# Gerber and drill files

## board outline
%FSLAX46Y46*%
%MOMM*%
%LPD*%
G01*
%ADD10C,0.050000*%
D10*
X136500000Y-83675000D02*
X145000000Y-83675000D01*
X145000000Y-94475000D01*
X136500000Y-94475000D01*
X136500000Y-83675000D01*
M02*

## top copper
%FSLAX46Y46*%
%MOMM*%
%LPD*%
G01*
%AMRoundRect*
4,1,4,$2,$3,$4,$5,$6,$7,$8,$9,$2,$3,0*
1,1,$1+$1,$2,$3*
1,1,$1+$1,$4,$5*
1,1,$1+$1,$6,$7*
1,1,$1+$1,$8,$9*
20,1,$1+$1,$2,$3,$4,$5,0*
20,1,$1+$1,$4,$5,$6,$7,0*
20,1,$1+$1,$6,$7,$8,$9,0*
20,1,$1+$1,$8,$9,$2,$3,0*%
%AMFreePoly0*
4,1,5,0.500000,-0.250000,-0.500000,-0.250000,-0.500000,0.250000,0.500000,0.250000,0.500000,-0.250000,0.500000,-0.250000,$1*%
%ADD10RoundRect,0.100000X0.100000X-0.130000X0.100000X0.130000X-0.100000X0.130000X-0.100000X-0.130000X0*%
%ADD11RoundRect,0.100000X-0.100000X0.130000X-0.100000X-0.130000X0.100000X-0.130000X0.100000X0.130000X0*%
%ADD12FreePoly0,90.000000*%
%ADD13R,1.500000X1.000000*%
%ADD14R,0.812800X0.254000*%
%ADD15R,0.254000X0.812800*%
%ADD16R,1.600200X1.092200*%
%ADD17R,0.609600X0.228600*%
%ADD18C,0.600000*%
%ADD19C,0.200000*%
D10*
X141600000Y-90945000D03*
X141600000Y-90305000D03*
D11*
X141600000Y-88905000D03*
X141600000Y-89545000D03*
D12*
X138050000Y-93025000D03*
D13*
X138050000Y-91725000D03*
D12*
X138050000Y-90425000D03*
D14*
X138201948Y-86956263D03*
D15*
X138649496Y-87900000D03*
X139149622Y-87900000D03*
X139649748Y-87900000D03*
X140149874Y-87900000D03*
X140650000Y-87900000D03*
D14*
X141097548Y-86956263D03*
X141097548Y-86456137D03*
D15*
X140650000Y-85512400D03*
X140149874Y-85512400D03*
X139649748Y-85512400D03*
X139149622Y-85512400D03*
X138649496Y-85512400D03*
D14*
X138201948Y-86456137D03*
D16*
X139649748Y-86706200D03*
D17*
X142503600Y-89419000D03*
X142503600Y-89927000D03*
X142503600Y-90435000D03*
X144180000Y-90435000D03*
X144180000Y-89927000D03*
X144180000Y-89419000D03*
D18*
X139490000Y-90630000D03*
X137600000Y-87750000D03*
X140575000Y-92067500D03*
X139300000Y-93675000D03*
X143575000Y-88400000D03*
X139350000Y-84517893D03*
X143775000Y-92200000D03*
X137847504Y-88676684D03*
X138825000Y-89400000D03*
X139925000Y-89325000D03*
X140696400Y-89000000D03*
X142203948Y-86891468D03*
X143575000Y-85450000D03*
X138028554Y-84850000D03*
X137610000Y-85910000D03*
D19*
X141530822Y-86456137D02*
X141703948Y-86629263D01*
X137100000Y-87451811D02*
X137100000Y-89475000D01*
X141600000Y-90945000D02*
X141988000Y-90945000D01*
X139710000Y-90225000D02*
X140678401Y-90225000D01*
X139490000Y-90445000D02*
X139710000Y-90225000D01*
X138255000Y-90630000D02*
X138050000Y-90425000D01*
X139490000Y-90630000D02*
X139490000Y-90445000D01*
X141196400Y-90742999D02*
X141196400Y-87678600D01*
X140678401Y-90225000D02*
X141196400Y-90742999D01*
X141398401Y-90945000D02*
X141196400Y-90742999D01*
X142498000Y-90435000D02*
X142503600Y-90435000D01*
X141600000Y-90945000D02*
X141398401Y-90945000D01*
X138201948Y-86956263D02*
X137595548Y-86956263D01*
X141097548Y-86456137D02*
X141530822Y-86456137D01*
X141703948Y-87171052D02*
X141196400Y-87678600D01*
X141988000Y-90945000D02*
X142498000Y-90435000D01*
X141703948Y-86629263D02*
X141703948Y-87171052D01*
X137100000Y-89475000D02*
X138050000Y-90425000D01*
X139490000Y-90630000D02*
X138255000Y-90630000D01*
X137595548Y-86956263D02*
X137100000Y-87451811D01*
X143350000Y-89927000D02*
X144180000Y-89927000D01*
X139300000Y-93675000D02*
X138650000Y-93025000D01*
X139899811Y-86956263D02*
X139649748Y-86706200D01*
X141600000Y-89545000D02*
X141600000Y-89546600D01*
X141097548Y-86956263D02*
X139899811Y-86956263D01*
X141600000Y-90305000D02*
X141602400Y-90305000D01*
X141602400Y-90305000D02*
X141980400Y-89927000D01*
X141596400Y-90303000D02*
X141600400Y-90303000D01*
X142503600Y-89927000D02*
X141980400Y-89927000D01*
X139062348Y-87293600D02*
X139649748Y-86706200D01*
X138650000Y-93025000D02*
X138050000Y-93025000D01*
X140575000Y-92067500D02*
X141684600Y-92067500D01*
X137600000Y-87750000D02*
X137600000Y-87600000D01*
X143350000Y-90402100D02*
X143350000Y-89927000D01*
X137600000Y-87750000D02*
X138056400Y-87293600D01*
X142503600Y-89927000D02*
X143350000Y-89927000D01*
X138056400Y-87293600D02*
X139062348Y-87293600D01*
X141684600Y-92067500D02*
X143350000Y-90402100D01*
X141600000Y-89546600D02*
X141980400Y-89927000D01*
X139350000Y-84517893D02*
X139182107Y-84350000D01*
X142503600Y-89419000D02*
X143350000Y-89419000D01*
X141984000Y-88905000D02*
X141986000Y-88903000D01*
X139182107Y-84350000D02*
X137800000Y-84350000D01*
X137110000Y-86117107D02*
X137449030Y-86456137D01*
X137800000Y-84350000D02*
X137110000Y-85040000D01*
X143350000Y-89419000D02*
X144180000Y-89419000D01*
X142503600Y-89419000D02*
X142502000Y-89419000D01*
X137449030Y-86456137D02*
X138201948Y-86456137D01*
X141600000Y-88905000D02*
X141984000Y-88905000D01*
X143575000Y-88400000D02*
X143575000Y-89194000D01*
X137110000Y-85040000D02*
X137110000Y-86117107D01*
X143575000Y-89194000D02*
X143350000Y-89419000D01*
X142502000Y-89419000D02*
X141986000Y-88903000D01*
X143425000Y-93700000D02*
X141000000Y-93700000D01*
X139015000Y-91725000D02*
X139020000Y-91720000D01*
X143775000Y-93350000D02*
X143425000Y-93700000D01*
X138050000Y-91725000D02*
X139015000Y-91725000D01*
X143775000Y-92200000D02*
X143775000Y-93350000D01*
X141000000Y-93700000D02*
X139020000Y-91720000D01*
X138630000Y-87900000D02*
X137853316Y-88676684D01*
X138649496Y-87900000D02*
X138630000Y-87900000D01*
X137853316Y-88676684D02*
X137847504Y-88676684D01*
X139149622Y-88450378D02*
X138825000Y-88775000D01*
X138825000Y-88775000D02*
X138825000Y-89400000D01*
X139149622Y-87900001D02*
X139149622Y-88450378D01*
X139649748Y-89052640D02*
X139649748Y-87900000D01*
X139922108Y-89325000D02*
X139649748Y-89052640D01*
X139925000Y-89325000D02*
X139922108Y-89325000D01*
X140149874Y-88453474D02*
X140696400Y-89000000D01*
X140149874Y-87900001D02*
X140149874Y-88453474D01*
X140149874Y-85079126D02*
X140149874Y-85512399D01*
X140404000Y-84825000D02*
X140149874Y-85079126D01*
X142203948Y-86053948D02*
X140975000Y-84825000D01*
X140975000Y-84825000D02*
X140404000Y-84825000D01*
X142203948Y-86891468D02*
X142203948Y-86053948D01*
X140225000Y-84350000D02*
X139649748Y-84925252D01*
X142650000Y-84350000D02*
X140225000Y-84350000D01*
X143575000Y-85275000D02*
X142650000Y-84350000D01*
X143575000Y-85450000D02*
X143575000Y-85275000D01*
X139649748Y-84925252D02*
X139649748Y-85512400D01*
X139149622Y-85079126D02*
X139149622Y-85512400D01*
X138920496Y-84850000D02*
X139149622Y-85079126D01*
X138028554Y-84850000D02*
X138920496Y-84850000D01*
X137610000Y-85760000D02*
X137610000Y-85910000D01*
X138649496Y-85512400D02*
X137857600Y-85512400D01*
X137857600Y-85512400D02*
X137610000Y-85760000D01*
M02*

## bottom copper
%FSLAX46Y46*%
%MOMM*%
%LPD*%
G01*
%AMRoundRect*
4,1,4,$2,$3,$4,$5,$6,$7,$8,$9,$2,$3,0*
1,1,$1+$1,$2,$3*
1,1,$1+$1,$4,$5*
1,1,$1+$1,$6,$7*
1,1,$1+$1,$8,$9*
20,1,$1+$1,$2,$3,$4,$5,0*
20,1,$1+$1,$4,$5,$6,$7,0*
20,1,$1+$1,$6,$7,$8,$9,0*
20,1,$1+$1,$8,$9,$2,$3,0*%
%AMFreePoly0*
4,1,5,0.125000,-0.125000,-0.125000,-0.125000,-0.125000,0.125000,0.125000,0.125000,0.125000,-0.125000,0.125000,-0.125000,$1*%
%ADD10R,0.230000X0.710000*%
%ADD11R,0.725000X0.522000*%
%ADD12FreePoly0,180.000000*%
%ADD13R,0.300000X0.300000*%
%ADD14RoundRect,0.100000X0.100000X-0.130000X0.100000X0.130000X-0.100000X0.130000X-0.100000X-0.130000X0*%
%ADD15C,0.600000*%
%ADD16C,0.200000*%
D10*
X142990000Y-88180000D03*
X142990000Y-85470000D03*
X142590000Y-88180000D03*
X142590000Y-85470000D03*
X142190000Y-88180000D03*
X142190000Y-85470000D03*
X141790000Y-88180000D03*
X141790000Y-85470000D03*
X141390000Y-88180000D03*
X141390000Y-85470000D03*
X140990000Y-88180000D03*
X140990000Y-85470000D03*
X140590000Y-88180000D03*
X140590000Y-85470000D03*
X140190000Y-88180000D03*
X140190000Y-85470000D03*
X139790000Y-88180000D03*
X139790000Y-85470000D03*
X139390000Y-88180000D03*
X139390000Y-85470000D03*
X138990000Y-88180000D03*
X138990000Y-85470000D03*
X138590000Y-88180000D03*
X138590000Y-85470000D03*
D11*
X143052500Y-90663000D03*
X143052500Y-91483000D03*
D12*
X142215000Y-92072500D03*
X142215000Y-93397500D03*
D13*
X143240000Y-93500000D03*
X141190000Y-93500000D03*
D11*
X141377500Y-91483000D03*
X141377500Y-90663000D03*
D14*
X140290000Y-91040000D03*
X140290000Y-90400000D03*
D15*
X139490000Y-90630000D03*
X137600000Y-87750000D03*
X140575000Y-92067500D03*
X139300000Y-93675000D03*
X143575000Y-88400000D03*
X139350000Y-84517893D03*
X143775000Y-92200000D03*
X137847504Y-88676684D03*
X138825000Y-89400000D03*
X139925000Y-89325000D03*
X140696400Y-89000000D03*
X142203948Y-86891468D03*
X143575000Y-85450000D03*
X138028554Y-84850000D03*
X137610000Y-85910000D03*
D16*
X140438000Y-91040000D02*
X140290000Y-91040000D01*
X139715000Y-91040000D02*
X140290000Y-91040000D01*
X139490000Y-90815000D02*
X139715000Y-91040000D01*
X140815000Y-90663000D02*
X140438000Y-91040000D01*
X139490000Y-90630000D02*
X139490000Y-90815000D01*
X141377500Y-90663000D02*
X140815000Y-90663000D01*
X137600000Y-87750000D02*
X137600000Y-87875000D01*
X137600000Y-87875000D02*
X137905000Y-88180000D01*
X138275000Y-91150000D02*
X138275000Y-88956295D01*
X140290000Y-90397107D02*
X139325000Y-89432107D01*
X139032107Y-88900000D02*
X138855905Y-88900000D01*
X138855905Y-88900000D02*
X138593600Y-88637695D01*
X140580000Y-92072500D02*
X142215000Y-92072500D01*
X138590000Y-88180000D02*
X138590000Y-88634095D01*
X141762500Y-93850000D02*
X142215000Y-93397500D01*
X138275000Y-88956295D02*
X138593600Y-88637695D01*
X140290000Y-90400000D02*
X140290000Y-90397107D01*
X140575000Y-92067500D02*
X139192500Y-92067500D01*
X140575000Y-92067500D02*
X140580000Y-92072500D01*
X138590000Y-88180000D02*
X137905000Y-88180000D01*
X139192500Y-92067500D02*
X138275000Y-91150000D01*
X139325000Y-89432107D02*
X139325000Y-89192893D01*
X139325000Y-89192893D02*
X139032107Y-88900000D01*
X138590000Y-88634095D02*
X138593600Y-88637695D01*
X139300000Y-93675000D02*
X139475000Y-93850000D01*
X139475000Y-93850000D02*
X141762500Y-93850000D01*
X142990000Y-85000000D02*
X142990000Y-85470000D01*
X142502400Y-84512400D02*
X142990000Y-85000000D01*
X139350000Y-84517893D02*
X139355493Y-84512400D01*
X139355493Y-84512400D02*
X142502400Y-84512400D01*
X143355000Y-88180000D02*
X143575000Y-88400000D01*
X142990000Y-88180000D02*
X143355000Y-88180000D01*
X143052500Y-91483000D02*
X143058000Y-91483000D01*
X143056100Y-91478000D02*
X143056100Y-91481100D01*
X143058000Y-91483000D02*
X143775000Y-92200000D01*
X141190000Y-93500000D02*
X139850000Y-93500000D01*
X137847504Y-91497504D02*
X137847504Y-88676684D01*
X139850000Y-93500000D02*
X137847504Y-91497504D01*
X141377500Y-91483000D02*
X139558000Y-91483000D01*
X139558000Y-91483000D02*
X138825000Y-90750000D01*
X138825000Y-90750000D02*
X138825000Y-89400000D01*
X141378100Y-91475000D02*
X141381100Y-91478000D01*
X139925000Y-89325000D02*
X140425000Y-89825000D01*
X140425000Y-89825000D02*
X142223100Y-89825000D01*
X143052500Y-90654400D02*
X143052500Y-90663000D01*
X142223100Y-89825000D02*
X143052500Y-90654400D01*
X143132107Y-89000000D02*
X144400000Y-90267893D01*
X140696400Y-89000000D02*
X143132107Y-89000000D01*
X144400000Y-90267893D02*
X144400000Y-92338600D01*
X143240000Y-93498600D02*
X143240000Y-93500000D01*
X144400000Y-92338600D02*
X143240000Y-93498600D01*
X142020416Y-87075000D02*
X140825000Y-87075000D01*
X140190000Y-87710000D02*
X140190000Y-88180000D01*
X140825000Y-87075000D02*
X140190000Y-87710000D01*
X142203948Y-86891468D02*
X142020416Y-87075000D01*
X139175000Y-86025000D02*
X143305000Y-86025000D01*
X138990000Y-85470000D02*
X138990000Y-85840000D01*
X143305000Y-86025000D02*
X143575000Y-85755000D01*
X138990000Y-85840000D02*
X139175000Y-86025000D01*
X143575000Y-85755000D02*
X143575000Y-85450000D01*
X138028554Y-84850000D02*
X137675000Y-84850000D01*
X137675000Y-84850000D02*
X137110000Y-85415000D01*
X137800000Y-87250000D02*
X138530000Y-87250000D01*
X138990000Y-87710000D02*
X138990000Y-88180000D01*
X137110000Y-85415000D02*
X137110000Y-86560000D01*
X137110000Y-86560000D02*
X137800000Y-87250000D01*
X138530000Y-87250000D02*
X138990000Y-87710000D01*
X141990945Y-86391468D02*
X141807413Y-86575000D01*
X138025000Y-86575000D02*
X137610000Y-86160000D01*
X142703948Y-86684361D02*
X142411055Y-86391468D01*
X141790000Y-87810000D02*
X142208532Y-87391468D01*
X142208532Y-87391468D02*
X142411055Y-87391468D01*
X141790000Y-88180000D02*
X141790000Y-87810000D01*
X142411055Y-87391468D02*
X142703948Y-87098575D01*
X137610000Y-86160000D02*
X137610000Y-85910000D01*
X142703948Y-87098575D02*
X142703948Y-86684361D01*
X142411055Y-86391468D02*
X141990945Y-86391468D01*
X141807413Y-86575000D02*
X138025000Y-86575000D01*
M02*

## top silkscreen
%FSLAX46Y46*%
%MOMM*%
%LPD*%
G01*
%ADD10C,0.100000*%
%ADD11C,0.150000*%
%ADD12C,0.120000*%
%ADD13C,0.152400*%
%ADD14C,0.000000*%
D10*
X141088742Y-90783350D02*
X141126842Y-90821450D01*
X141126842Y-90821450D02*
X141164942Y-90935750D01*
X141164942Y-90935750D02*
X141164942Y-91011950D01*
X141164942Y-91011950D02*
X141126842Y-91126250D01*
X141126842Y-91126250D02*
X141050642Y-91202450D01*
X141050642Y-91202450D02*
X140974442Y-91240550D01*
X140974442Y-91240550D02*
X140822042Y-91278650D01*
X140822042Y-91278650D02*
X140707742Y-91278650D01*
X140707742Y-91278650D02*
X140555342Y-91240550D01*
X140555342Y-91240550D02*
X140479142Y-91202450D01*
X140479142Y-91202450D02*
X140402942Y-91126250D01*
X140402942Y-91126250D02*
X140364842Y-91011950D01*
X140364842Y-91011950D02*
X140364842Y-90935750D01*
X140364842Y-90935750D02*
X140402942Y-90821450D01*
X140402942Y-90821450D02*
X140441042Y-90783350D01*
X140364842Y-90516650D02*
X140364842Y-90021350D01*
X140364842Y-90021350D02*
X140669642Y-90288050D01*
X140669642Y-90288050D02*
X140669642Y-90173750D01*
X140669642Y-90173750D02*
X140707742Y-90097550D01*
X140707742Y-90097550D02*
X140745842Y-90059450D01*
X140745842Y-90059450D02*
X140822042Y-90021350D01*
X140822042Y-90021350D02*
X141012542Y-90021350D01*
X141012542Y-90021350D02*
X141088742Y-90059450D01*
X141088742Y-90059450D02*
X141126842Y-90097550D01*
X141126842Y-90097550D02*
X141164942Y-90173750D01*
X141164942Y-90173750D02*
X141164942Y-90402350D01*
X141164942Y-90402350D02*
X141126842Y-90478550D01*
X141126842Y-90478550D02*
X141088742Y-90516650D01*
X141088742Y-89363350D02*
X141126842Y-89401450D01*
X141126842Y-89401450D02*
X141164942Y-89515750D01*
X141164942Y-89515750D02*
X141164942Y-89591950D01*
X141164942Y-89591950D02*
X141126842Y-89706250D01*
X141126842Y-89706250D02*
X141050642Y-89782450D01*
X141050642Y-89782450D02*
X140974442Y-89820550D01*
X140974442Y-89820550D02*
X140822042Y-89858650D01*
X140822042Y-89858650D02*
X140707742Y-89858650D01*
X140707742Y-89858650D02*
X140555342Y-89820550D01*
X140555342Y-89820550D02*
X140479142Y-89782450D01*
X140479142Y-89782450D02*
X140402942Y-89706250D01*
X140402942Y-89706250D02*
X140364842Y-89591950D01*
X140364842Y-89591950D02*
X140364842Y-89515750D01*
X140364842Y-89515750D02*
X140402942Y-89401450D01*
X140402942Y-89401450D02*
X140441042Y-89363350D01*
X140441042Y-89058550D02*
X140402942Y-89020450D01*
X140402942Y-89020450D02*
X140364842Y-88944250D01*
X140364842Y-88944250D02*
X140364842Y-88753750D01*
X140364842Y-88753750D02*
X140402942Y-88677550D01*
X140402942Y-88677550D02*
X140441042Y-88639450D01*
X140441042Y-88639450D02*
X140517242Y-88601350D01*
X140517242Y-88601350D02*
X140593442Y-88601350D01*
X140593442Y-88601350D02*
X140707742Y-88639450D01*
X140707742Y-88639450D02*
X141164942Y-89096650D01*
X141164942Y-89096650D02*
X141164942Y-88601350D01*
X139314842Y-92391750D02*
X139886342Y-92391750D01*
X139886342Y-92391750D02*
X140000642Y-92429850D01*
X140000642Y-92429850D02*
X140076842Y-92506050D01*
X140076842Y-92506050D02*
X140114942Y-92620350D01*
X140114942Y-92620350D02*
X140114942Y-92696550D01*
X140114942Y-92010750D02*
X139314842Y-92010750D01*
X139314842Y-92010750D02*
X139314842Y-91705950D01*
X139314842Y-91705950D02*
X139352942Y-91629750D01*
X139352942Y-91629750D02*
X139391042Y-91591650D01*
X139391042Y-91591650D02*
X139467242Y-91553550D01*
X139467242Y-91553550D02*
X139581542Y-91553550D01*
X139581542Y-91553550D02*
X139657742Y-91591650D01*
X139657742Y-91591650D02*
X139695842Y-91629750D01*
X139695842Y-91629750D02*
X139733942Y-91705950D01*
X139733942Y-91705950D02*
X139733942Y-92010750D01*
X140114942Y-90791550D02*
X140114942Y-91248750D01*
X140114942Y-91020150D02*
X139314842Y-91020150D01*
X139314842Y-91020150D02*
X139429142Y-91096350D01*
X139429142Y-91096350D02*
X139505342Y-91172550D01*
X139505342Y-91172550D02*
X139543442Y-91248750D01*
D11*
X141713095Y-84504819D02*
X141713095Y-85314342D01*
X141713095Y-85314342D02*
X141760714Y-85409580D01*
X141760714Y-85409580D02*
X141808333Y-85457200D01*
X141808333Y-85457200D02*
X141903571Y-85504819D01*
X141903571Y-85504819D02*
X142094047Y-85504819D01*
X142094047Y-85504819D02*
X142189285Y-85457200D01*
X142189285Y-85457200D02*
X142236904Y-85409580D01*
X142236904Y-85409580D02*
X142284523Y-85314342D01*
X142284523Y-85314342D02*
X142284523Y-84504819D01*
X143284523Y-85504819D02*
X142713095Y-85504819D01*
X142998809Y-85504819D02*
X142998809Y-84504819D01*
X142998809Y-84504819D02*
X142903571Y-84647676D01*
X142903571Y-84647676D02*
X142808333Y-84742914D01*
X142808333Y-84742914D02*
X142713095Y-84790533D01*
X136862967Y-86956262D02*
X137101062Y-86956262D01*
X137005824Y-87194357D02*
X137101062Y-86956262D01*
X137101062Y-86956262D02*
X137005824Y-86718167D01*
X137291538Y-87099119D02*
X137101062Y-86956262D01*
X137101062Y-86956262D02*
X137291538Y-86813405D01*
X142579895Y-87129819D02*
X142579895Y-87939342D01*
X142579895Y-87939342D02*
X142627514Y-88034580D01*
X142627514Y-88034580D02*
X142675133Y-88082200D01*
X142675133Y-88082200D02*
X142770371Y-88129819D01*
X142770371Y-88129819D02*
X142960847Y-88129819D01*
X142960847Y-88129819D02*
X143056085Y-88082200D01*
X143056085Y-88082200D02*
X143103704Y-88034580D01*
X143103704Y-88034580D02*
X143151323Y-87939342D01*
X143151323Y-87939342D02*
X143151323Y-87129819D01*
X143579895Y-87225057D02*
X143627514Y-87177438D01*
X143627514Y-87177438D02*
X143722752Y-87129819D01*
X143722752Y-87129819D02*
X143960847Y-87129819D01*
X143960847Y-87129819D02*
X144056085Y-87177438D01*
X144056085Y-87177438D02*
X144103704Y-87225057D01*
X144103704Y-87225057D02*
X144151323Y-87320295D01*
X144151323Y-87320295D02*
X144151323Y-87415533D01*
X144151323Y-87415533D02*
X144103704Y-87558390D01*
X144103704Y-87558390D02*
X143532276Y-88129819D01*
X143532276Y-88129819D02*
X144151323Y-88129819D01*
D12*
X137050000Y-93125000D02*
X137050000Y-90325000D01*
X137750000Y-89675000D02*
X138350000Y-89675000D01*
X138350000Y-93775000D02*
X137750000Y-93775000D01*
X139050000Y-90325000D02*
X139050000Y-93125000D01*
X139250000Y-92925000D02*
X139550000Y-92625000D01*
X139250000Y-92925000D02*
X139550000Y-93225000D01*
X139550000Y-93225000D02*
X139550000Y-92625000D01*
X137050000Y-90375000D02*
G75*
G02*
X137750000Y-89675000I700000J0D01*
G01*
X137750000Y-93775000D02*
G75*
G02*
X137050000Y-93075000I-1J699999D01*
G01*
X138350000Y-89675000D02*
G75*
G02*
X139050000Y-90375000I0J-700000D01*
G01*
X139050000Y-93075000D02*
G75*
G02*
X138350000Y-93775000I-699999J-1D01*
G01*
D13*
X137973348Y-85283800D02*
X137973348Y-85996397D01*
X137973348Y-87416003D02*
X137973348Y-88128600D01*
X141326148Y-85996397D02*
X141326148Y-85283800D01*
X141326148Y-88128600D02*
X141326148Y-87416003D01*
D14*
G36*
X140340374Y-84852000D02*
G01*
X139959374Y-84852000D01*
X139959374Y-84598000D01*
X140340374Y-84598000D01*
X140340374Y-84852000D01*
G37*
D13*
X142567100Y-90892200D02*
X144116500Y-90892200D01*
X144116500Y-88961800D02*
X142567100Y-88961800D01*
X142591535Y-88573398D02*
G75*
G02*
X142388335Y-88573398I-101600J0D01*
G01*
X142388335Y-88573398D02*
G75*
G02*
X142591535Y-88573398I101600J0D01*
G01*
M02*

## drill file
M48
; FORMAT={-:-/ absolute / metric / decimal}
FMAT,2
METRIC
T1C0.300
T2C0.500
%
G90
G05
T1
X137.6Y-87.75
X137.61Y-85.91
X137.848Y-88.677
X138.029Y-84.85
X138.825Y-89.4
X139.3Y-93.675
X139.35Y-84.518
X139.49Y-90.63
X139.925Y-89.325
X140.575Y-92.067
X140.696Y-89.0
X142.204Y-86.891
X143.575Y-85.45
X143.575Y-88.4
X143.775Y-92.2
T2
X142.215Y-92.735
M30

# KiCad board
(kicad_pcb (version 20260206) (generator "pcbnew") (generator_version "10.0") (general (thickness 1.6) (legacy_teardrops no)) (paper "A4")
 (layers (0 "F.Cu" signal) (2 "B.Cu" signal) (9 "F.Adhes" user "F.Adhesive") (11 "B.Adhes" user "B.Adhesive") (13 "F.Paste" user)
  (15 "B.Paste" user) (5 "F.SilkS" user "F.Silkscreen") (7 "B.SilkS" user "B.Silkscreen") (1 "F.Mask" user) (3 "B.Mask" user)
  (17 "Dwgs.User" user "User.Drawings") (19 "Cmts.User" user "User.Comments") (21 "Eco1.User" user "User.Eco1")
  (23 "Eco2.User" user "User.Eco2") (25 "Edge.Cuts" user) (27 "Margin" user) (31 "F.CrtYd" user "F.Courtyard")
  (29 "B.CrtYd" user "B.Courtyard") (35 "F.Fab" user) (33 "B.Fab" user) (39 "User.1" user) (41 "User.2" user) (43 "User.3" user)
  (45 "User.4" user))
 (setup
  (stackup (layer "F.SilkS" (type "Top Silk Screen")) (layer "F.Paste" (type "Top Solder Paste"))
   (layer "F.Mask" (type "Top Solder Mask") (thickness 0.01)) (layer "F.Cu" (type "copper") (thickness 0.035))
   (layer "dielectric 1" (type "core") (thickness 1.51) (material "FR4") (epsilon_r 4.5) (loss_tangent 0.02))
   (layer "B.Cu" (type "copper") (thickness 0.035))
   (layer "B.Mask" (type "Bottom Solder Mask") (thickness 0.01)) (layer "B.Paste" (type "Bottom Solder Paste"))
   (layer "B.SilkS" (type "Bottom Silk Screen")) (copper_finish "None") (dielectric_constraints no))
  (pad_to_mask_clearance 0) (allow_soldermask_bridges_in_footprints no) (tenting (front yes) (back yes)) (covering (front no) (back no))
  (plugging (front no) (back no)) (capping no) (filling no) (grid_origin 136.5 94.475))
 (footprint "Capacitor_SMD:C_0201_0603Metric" (layer "F.Cu") (at 141.6 90.625 90)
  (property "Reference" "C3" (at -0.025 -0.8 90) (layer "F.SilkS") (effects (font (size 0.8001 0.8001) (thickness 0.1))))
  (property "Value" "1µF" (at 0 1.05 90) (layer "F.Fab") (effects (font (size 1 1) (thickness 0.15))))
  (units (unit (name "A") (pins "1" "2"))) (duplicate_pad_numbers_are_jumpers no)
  (pad "" smd roundrect (at -0.345 0 90) (size 0.318 0.36) (layers "F.Paste") (roundrect_rratio 0.25))
  (pad "" smd roundrect (at 0.345 0 90) (size 0.318 0.36) (layers "F.Paste") (roundrect_rratio 0.25))
  (pad "1" smd roundrect (at -0.32 0 90) (size 0.46 0.4) (layers "F.Cu" "F.Mask") (roundrect_rratio 0.25) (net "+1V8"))
  (pad "2" smd roundrect (at 0.32 0 90) (size 0.46 0.4) (layers "F.Cu" "F.Mask") (roundrect_rratio 0.25) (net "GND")))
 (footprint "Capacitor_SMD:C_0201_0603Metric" (layer "F.Cu") (at 141.6 89.225 -90)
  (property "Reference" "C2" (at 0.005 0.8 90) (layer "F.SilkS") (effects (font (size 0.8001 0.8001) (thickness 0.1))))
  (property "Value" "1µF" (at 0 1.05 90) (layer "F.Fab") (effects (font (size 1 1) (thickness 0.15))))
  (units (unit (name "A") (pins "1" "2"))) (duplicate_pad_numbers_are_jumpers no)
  (pad "" smd roundrect (at -0.345 0 270) (size 0.318 0.36) (layers "F.Paste") (roundrect_rratio 0.25))
  (pad "" smd roundrect (at 0.345 0 270) (size 0.318 0.36) (layers "F.Paste") (roundrect_rratio 0.25))
  (pad "1" smd roundrect (at -0.32 0 270) (size 0.46 0.4) (layers "F.Cu" "F.Mask") (roundrect_rratio 0.25) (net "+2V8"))
  (pad "2" smd roundrect (at 0.32 0 270) (size 0.46 0.4) (layers "F.Cu" "F.Mask") (roundrect_rratio 0.25) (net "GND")))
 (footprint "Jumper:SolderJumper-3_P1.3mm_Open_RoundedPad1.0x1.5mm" (layer "F.Cu") (at 138.05 91.725 90)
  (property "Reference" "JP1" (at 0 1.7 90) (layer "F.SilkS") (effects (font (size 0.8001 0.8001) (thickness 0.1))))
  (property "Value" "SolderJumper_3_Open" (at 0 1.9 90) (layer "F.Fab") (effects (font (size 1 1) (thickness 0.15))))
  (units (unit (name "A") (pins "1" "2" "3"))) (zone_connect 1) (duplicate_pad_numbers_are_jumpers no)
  (fp_line (start -1.4 -1) (end 1.4 -1) (stroke (width 0.12) (type solid)) (layer "F.SilkS"))
  (fp_line (start 2.05 -0.3) (end 2.05 0.3) (stroke (width 0.12) (type solid)) (layer "F.SilkS"))
  (fp_line (start -2.05 0.3) (end -2.05 -0.3) (stroke (width 0.12) (type solid)) (layer "F.SilkS"))
  (fp_line (start 1.4 1) (end -1.4 1) (stroke (width 0.12) (type solid)) (layer "F.SilkS"))
  (fp_line (start -1.2 1.2) (end -0.9 1.5) (stroke (width 0.12) (type solid)) (layer "F.SilkS"))
  (fp_line (start -1.2 1.2) (end -1.5 1.5) (stroke (width 0.12) (type solid)) (layer "F.SilkS"))
  (fp_line (start -1.5 1.5) (end -0.9 1.5) (stroke (width 0.12) (type solid)) (layer "F.SilkS"))
  (fp_arc (start 1.35 -1) (mid 1.844975 -0.794975) (end 2.05 -0.3) (stroke (width 0.12) (type solid)) (layer "F.SilkS"))
  (fp_arc (start -2.05 -0.3) (mid -1.844975 -0.794975) (end -1.35 -1) (stroke (width 0.12) (type solid)) (layer "F.SilkS"))
  (fp_arc (start 2.05 0.3) (mid 1.844975 0.794975) (end 1.35 1) (stroke (width 0.12) (type solid)) (layer "F.SilkS"))
  (fp_arc (start -1.35 1) (mid -1.844975 0.794975) (end -2.05 0.3) (stroke (width 0.12) (type solid)) (layer "F.SilkS"))
  (pad "1" smd custom (at -1.3 0 90) (size 1 0.5) (layers "F.Cu" "F.Mask") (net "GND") (zone_connect 2) (thermal_bridge_angle 45)
   (options (clearance outline) (anchor rect)) (primitives))
  (pad "2" smd rect (at 0 0 90) (size 1 1.5) (layers "F.Cu" "F.Mask") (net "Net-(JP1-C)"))
  (pad "3" smd custom (at 1.3 0 90) (size 1 0.5) (layers "F.Cu" "F.Mask") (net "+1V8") (zone_connect 2) (thermal_bridge_angle 45)
   (options (clearance outline) (anchor rect)) (primitives)))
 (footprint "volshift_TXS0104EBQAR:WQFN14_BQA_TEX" (layer "F.Cu") (at 139.649748 86.7062 90)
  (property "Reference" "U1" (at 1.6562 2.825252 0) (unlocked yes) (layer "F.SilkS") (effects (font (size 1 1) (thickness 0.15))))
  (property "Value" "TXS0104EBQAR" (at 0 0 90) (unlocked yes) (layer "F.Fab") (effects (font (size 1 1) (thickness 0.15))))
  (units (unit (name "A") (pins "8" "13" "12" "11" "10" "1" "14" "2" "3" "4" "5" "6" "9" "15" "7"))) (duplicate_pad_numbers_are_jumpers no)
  (fp_line (start 1.4224 -1.6764) (end 0.709803 -1.6764) (stroke (width 0.1524) (type solid)) (layer "F.SilkS"))
  (fp_line (start -0.709803 -1.6764) (end -1.4224 -1.6764) (stroke (width 0.1524) (type solid)) (layer "F.SilkS"))
  (fp_line (start 0.709803 1.6764) (end 1.4224 1.6764) (stroke (width 0.1524) (type solid)) (layer "F.SilkS"))
  (fp_line (start -1.4224 1.6764) (end -0.709803 1.6764) (stroke (width 0.1524) (type solid)) (layer "F.SilkS"))
  (fp_poly
   (pts (xy 2.1082 0.309626) (xy 2.1082 0.690626) (xy 1.8542 0.690626) (xy 1.8542 0.309626)) (stroke (width 0) (type solid)) (fill yes)
   (layer "F.SilkS"))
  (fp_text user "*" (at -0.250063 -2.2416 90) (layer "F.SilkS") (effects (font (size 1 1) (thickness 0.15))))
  (pad "1" smd rect (at -0.250063 -1.4478 90) (size 0.254 0.8128) (layers "F.Cu" "F.Mask" "F.Paste") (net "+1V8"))
  (pad "2" smd rect (at -1.1938 -1.000252 180) (size 0.254 0.8128) (layers "F.Cu" "F.Mask" "F.Paste") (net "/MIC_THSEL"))
  (pad "3" smd rect (at -1.1938 -0.500126 180) (size 0.254 0.8128) (layers "F.Cu" "F.Mask" "F.Paste") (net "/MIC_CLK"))
  (pad "4" smd rect (at -1.1938 0 180) (size 0.254 0.8128) (layers "F.Cu" "F.Mask" "F.Paste") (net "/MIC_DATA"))
  (pad "5" smd rect (at -1.1938 0.500126 180) (size 0.254 0.8128) (layers "F.Cu" "F.Mask" "F.Paste") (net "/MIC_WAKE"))
  (pad "6" smd rect (at -1.1938 1.000252 180) (size 0.254 0.8128) (layers "F.Cu" "F.Mask" "F.Paste") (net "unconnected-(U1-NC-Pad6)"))
  (pad "7" smd rect (at -0.250063 1.4478 90) (size 0.254 0.8128) (layers "F.Cu" "F.Mask" "F.Paste") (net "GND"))
  (pad "8" smd rect (at 0.250063 1.4478 90) (size 0.254 0.8128) (layers "F.Cu" "F.Mask" "F.Paste") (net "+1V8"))
  (pad "9" smd rect (at 1.1938 1.000252 180) (size 0.254 0.8128) (layers "F.Cu" "F.Mask" "F.Paste") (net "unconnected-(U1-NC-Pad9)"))
  (pad "10" smd rect (at 1.1938 0.500126 180) (size 0.254 0.8128) (layers "F.Cu" "F.Mask" "F.Paste") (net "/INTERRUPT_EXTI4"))
  (pad "11" smd rect (at 1.1938 0 180) (size 0.254 0.8128) (layers "F.Cu" "F.Mask" "F.Paste") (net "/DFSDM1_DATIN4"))
  (pad "12" smd rect (at 1.1938 -0.500126 180) (size 0.254 0.8128) (layers "F.Cu" "F.Mask" "F.Paste") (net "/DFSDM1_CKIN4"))
  (pad "13" smd rect (at 1.1938 -1.000252 180) (size 0.254 0.8128) (layers "F.Cu" "F.Mask" "F.Paste") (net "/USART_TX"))
  (pad "14" smd rect (at 0.250063 -1.4478 90) (size 0.254 0.8128) (layers "F.Cu" "F.Mask" "F.Paste") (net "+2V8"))
  (pad "15" smd rect (at 0 0 90) (size 1.0922 1.6002) (layers "F.Cu" "F.Mask" "F.Paste") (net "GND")))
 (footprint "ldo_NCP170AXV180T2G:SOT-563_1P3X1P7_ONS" (layer "F.Cu") (at 143.3418 89.927)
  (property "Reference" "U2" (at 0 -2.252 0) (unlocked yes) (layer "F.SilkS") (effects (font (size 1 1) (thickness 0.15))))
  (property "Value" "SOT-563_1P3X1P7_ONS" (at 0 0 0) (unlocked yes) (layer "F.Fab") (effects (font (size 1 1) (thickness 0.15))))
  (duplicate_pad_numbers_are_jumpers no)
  (fp_line (start -0.7747 0.9652) (end 0.7747 0.9652) (stroke (width 0.1524) (type solid)) (layer "F.SilkS"))
  (fp_line (start 0.7747 -0.9652) (end -0.7747 -0.9652) (stroke (width 0.1524) (type solid)) (layer "F.SilkS"))
  (fp_circle (center -0.851865 -1.353602) (end -0.750265 -1.353602) (stroke (width 0.1524) (type solid)) (fill no) (layer "F.SilkS"))
  (pad "1" smd rect (at -0.8382 -0.508) (size 0.6096 0.2286) (layers "F.Cu" "F.Mask" "F.Paste") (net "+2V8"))
  (pad "2" smd rect (at -0.8382 0) (size 0.6096 0.2286) (layers "F.Cu" "F.Mask" "F.Paste") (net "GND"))
  (pad "3" smd rect (at -0.8382 0.508) (size 0.6096 0.2286) (layers "F.Cu" "F.Mask" "F.Paste") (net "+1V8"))
  (pad "4" smd rect (at 0.8382 0.508) (size 0.6096 0.2286) (layers "F.Cu" "F.Mask" "F.Paste") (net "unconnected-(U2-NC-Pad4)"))
  (pad "5" smd rect (at 0.8382 0) (size 0.6096 0.2286) (layers "F.Cu" "F.Mask" "F.Paste") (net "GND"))
  (pad "6" smd rect (at 0.8382 -0.508) (size 0.6096 0.2286) (layers "F.Cu" "F.Mask" "F.Paste") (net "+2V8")))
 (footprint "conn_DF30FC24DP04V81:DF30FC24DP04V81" (layer "B.Cu") (at 140.79 86.825 180)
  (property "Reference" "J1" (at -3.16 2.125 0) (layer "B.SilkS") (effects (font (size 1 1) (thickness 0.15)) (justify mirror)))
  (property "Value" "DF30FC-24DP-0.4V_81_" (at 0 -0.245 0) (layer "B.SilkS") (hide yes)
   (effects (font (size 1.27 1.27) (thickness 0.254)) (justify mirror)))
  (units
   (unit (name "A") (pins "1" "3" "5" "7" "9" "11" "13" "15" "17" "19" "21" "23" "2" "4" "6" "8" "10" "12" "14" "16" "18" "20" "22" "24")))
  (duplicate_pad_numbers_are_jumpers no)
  (pad "1" smd rect (at -2.2 -1.355 180) (size 0.23 0.71) (layers "B.Cu" "B.Mask" "B.Paste") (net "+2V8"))
  (pad "2" smd rect (at -2.2 1.355 180) (size 0.23 0.71) (layers "B.Cu" "B.Mask" "B.Paste") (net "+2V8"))
  (pad "3" smd rect (at -1.8 -1.355 180) (size 0.23 0.71) (layers "B.Cu" "B.Mask" "B.Paste") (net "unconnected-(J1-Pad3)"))
  (pad "4" smd rect (at -1.8 1.355 180) (size 0.23 0.71) (layers "B.Cu" "B.Mask" "B.Paste") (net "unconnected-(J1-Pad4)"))
  (pad "5" smd rect (at -1.4 -1.355 180) (size 0.23 0.71) (layers "B.Cu" "B.Mask" "B.Paste") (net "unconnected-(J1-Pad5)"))
  (pad "6" smd rect (at -1.4 1.355 180) (size 0.23 0.71) (layers "B.Cu" "B.Mask" "B.Paste") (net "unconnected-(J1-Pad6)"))
  (pad "7" smd rect (at -1 -1.355 180) (size 0.23 0.71) (layers "B.Cu" "B.Mask" "B.Paste") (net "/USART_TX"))
  (pad "8" smd rect (at -1 1.355 180) (size 0.23 0.71) (layers "B.Cu" "B.Mask" "B.Paste") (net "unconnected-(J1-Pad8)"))
  (pad "9" smd rect (at -0.6 -1.355 180) (size 0.23 0.71) (layers "B.Cu" "B.Mask" "B.Paste") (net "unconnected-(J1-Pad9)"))
  (pad "10" smd rect (at -0.6 1.355 180) (size 0.23 0.71) (layers "B.Cu" "B.Mask" "B.Paste") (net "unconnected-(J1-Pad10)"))
  (pad "11" smd rect (at -0.2 -1.355 180) (size 0.23 0.71) (layers "B.Cu" "B.Mask" "B.Paste") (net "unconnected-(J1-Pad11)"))
  (pad "12" smd rect (at -0.2 1.355 180) (size 0.23 0.71) (layers "B.Cu" "B.Mask" "B.Paste") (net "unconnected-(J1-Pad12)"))
  (pad "13" smd rect (at 0.2 -1.355 180) (size 0.23 0.71) (layers "B.Cu" "B.Mask" "B.Paste") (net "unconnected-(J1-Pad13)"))
  (pad "14" smd rect (at 0.2 1.355 180) (size 0.23 0.71) (layers "B.Cu" "B.Mask" "B.Paste") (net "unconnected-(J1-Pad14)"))
  (pad "15" smd rect (at 0.6 -1.355 180) (size 0.23 0.71) (layers "B.Cu" "B.Mask" "B.Paste") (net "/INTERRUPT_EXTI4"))
  (pad "16" smd rect (at 0.6 1.355 180) (size 0.23 0.71) (layers "B.Cu" "B.Mask" "B.Paste") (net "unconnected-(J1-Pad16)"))
  (pad "17" smd rect (at 1 -1.355 180) (size 0.23 0.71) (layers "B.Cu" "B.Mask" "B.Paste") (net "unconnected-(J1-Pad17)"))
  (pad "18" smd rect (at 1 1.355 180) (size 0.23 0.71) (layers "B.Cu" "B.Mask" "B.Paste") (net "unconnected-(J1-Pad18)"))
  (pad "19" smd rect (at 1.4 -1.355 180) (size 0.23 0.71) (layers "B.Cu" "B.Mask" "B.Paste") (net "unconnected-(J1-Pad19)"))
  (pad "20" smd rect (at 1.4 1.355 180) (size 0.23 0.71) (layers "B.Cu" "B.Mask" "B.Paste") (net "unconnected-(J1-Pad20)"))
  (pad "21" smd rect (at 1.8 -1.355 180) (size 0.23 0.71) (layers "B.Cu" "B.Mask" "B.Paste") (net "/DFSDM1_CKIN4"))
  (pad "22" smd rect (at 1.8 1.355 180) (size 0.23 0.71) (layers "B.Cu" "B.Mask" "B.Paste") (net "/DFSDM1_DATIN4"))
  (pad "23" smd rect (at 2.2 -1.355 180) (size 0.23 0.71) (layers "B.Cu" "B.Mask" "B.Paste") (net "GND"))
  (pad "24" smd rect (at 2.2 1.355 180) (size 0.23 0.71) (layers "B.Cu" "B.Mask" "B.Paste") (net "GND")))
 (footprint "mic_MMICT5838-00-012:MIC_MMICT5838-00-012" (layer "B.Cu") (at 142.215 92.025 180)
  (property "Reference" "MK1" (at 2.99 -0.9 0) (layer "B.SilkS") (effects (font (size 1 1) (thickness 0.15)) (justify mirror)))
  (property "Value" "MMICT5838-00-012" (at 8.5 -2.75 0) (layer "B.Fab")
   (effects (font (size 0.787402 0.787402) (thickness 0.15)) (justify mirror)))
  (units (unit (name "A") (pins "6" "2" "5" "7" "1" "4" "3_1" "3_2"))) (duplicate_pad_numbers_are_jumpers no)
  (pad "" np_thru_hole circle (at 0 -0.71 180) (size 0.5 0.5) (drill 0.5) (layers "*.Cu" "*.Mask"))
  (pad "1" smd rect (at -0.8375 1.362 180) (size 0.725 0.522) (layers "B.Cu") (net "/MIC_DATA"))
  (pad "2" smd rect (at -0.8375 0.542 180) (size 0.725 0.522) (layers "B.Cu") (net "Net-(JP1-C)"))
  (pad "3_1" smd custom (at 0 -0.0475 180) (size 0.25 0.25) (layers "B.Cu") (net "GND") (options (clearance outline) (anchor rect))
   (primitives))
  (pad "3_2" smd custom (at 0 -1.3725 180) (size 0.25 0.25) (layers "B.Cu") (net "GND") (options (clearance outline) (anchor rect))
   (primitives))
  (pad "4" smd rect (at -1.025 -1.475 180) (size 0.3 0.3) (layers "B.Cu") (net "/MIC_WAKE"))
  (pad "5" smd rect (at 1.025 -1.475 180) (size 0.3 0.3) (layers "B.Cu") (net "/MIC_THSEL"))
  (pad "6" smd rect (at 0.8375 0.542 180) (size 0.725 0.522) (layers "B.Cu") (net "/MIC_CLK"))
  (pad "7" smd rect (at 0.8375 1.362 180) (size 0.725 0.522) (layers "B.Cu") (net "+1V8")))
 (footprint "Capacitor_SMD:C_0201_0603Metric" (layer "B.Cu") (at 140.29 90.72 90)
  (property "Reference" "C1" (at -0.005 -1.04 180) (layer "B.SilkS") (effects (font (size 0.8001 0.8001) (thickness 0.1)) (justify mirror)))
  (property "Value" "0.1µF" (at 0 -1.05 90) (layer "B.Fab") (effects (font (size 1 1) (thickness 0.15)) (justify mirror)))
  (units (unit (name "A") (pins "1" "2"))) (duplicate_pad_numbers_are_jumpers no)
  (pad "" smd roundrect (at -0.345 0 90) (size 0.318 0.36) (layers "B.Paste") (roundrect_rratio 0.25))
  (pad "" smd roundrect (at 0.345 0 90) (size 0.318 0.36) (layers "B.Paste") (roundrect_rratio 0.25))
  (pad "1" smd roundrect (at -0.32 0 90) (size 0.46 0.4) (layers "B.Cu" "B.Mask") (roundrect_rratio 0.25) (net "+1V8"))
  (pad "2" smd roundrect (at 0.32 0 90) (size 0.46 0.4) (layers "B.Cu" "B.Mask") (roundrect_rratio 0.25) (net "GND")))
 (gr_rect (start 136.5 83.675) (end 145 94.475) (stroke (width 0.05) (type default)) (fill no) (layer "Edge.Cuts"))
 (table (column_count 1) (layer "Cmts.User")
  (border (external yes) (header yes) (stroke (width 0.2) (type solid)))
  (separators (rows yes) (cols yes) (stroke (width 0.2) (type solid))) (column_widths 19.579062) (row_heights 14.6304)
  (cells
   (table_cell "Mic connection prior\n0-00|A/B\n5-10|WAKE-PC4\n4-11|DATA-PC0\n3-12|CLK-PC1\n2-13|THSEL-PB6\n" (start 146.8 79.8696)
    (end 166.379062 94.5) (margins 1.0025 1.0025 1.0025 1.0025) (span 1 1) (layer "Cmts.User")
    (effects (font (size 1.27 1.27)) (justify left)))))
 (segment (start 141.530822 86.456137) (end 141.703948 86.629263) (width 0.2) (layer "F.Cu") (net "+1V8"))
 (segment (start 137.1 87.451811) (end 137.1 89.475) (width 0.2) (layer "F.Cu") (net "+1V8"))
 (segment (start 141.6 90.945) (end 141.988 90.945) (width 0.2) (layer "F.Cu") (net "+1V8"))
 (segment (start 139.71 90.225) (end 140.678401 90.225) (width 0.2) (layer "F.Cu") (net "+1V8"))
 (segment (start 139.49 90.445) (end 139.71 90.225) (width 0.2) (layer "F.Cu") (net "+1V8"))
 (segment (start 138.255 90.63) (end 138.05 90.425) (width 0.2) (layer "F.Cu") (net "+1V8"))
 (segment (start 139.49 90.63) (end 139.49 90.445) (width 0.2) (layer "F.Cu") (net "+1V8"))
 (segment (start 141.1964 90.742999) (end 141.1964 87.6786) (width 0.2) (layer "F.Cu") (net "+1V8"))
 (segment (start 140.678401 90.225) (end 141.1964 90.742999) (width 0.2) (layer "F.Cu") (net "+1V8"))
 (segment (start 141.398401 90.945) (end 141.1964 90.742999) (width 0.2) (layer "F.Cu") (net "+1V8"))
 (segment (start 142.498 90.435) (end 142.5036 90.435) (width 0.2) (layer "F.Cu") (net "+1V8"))
 (segment (start 141.6 90.945) (end 141.398401 90.945) (width 0.2) (layer "F.Cu") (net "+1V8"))
 (segment (start 138.201948 86.956263) (end 137.595548 86.956263) (width 0.2) (layer "F.Cu") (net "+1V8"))
 (segment (start 141.097548 86.456137) (end 141.530822 86.456137) (width 0.2) (layer "F.Cu") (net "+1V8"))
 (segment (start 141.703948 87.171052) (end 141.1964 87.6786) (width 0.2) (layer "F.Cu") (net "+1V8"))
 (segment (start 141.988 90.945) (end 142.498 90.435) (width 0.2) (layer "F.Cu") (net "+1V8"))
 (segment (start 141.703948 86.629263) (end 141.703948 87.171052) (width 0.2) (layer "F.Cu") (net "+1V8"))
 (segment (start 137.1 89.475) (end 138.05 90.425) (width 0.2) (layer "F.Cu") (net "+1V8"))
 (segment (start 139.49 90.63) (end 138.255 90.63) (width 0.2) (layer "F.Cu") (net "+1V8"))
 (segment (start 137.595548 86.956263) (end 137.1 87.451811) (width 0.2) (layer "F.Cu") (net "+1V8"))
 (via (at 139.49 90.63) (size 0.6) (drill 0.3) (layers "F.Cu" "B.Cu") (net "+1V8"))
 (segment (start 140.438 91.04) (end 140.29 91.04) (width 0.2) (layer "B.Cu") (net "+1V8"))
 (segment (start 139.715 91.04) (end 140.29 91.04) (width 0.2) (layer "B.Cu") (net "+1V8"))
 (segment (start 139.49 90.815) (end 139.715 91.04) (width 0.2) (layer "B.Cu") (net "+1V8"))
 (segment (start 140.815 90.663) (end 140.438 91.04) (width 0.2) (layer "B.Cu") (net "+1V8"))
 (segment (start 139.49 90.63) (end 139.49 90.815) (width 0.2) (layer "B.Cu") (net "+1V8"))
 (segment (start 141.3775 90.663) (end 140.815 90.663) (width 0.2) (layer "B.Cu") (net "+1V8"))
 (segment (start 143.35 89.927) (end 144.18 89.927) (width 0.2) (layer "F.Cu") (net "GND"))
 (segment (start 139.3 93.675) (end 138.65 93.025) (width 0.2) (layer "F.Cu") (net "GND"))
 (segment (start 139.899811 86.956263) (end 139.649748 86.7062) (width 0.2) (layer "F.Cu") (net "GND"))
 (segment (start 141.6 89.545) (end 141.6 89.5466) (width 0.2) (layer "F.Cu") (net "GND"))
 (segment (start 141.097548 86.956263) (end 139.899811 86.956263) (width 0.2) (layer "F.Cu") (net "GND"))
 (segment (start 141.6 90.305) (end 141.6024 90.305) (width 0.2) (layer "F.Cu") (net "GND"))
 (segment (start 141.6024 90.305) (end 141.9804 89.927) (width 0.2) (layer "F.Cu") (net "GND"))
 (segment (start 141.5964 90.303) (end 141.6004 90.303) (width 0.2) (layer "F.Cu") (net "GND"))
 (segment (start 142.5036 89.927) (end 141.9804 89.927) (width 0.2) (layer "F.Cu") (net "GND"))
 (segment (start 139.062348 87.2936) (end 139.649748 86.7062) (width 0.2) (layer "F.Cu") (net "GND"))
 (segment (start 138.65 93.025) (end 138.05 93.025) (width 0.2) (layer "F.Cu") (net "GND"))
 (segment (start 140.575 92.0675) (end 141.6846 92.0675) (width 0.2) (layer "F.Cu") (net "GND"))
 (segment (start 137.6 87.75) (end 137.6 87.6) (width 0.2) (layer "F.Cu") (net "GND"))
 (segment (start 143.35 90.4021) (end 143.35 89.927) (width 0.2) (layer "F.Cu") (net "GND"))
 (segment (start 137.6 87.75) (end 138.0564 87.2936) (width 0.2) (layer "F.Cu") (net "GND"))
 (segment (start 142.5036 89.927) (end 143.35 89.927) (width 0.2) (layer "F.Cu") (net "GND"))
 (segment (start 138.0564 87.2936) (end 139.062348 87.2936) (width 0.2) (layer "F.Cu") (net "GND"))
 (segment (start 141.6846 92.0675) (end 143.35 90.4021) (width 0.2) (layer "F.Cu") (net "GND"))
 (segment (start 141.6 89.5466) (end 141.9804 89.927) (width 0.2) (layer "F.Cu") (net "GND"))
 (via (at 137.6 87.75) (size 0.6) (drill 0.3) (layers "F.Cu" "B.Cu") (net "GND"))
 (via (at 140.575 92.0675) (size 0.6) (drill 0.3) (layers "F.Cu" "B.Cu") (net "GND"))
 (via (at 139.3 93.675) (size 0.6) (drill 0.3) (layers "F.Cu" "B.Cu") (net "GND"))
 (segment (start 137.6 87.75) (end 137.6 87.875) (width 0.2) (layer "B.Cu") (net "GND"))
 (segment (start 137.6 87.875) (end 137.905 88.18) (width 0.2) (layer "B.Cu") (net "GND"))
 (segment (start 138.275 91.15) (end 138.275 88.956295) (width 0.2) (layer "B.Cu") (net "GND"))
 (segment (start 140.29 90.397107) (end 139.325 89.432107) (width 0.2) (layer "B.Cu") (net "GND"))
 (segment (start 139.032107 88.9) (end 138.855905 88.9) (width 0.2) (layer "B.Cu") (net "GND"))
 (segment (start 138.855905 88.9) (end 138.5936 88.637695) (width 0.2) (layer "B.Cu") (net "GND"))
 (segment (start 140.58 92.0725) (end 142.215 92.0725) (width 0.2) (layer "B.Cu") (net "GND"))
 (segment (start 138.59 88.18) (end 138.59 88.634095) (width 0.2) (layer "B.Cu") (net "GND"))
 (segment (start 141.7625 93.85) (end 142.215 93.3975) (width 0.2) (layer "B.Cu") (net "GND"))
 (segment (start 138.275 88.956295) (end 138.5936 88.637695) (width 0.2) (layer "B.Cu") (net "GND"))
 (segment (start 140.29 90.4) (end 140.29 90.397107) (width 0.2) (layer "B.Cu") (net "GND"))
 (segment (start 140.575 92.0675) (end 139.1925 92.0675) (width 0.2) (layer "B.Cu") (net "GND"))
 (segment (start 140.575 92.0675) (end 140.58 92.0725) (width 0.2) (layer "B.Cu") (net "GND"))
 (segment (start 138.59 88.18) (end 137.905 88.18) (width 0.2) (layer "B.Cu") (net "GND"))
 (segment (start 139.1925 92.0675) (end 138.275 91.15) (width 0.2) (layer "B.Cu") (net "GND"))
 (segment (start 139.325 89.432107) (end 139.325 89.192893) (width 0.2) (layer "B.Cu") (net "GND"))
 (segment (start 139.325 89.192893) (end 139.032107 88.9) (width 0.2) (layer "B.Cu") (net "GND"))
 (segment (start 138.59 88.634095) (end 138.5936 88.637695) (width 0.2) (layer "B.Cu") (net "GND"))
 (segment (start 139.3 93.675) (end 139.475 93.85) (width 0.2) (layer "B.Cu") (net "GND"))
 (segment (start 139.475 93.85) (end 141.7625 93.85) (width 0.2) (layer "B.Cu") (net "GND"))
 (segment (start 139.35 84.517893) (end 139.182107 84.35) (width 0.2) (layer "F.Cu") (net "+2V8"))
 (segment (start 142.5036 89.419) (end 143.35 89.419) (width 0.2) (layer "F.Cu") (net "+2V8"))
 (segment (start 141.984 88.905) (end 141.986 88.903) (width 0.2) (layer "F.Cu") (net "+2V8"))
 (segment (start 139.182107 84.35) (end 137.8 84.35) (width 0.2) (layer "F.Cu") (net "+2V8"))
 (segment (start 137.11 86.117107) (end 137.44903 86.456137) (width 0.2) (layer "F.Cu") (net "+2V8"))
 (segment (start 137.8 84.35) (end 137.11 85.04) (width 0.2) (layer "F.Cu") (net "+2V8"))
 (segment (start 143.35 89.419) (end 144.18 89.419) (width 0.2) (layer "F.Cu") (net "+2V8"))
 (segment (start 142.5036 89.419) (end 142.502 89.419) (width 0.2) (layer "F.Cu") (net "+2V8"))
 (segment (start 137.44903 86.456137) (end 138.201948 86.456137) (width 0.2) (layer "F.Cu") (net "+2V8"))
 (segment (start 141.6 88.905) (end 141.984 88.905) (width 0.2) (layer "F.Cu") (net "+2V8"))
 (segment (start 143.575 88.4) (end 143.575 89.194) (width 0.2) (layer "F.Cu") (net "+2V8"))
 (segment (start 137.11 85.04) (end 137.11 86.117107) (width 0.2) (layer "F.Cu") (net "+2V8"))
 (segment (start 143.575 89.194) (end 143.35 89.419) (width 0.2) (layer "F.Cu") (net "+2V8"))
 (segment (start 142.502 89.419) (end 141.986 88.903) (width 0.2) (layer "F.Cu") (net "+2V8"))
 (via (at 143.575 88.4) (size 0.6) (drill 0.3) (layers "F.Cu" "B.Cu") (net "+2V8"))
 (via (at 139.35 84.517893) (size 0.6) (drill 0.3) (layers "F.Cu" "B.Cu") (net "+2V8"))
 (segment (start 142.99 85) (end 142.99 85.47) (width 0.2) (layer "B.Cu") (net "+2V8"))
 (segment (start 142.5024 84.5124) (end 142.99 85) (width 0.2) (layer "B.Cu") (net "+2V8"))
 (segment (start 139.35 84.517893) (end 139.355493 84.5124) (width 0.2) (layer "B.Cu") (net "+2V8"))
 (segment (start 139.355493 84.5124) (end 142.5024 84.5124) (width 0.2) (layer "B.Cu") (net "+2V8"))
 (segment (start 143.355 88.18) (end 143.575 88.4) (width 0.2) (layer "B.Cu") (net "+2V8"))
 (segment (start 142.99 88.18) (end 143.355 88.18) (width 0.2) (layer "B.Cu") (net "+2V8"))
 (segment (start 143.425 93.7) (end 141 93.7) (width 0.2) (layer "F.Cu") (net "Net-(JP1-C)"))
 (segment (start 139.015 91.725) (end 139.02 91.72) (width 0.2) (layer "F.Cu") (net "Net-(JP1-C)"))
 (segment (start 143.775 93.35) (end 143.425 93.7) (width 0.2) (layer "F.Cu") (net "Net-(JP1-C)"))
 (segment (start 138.05 91.725) (end 139.015 91.725) (width 0.2) (layer "F.Cu") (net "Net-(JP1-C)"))
 (segment (start 143.775 92.2) (end 143.775 93.35) (width 0.2) (layer "F.Cu") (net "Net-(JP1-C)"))
 (segment (start 141 93.7) (end 139.02 91.72) (width 0.2) (layer "F.Cu") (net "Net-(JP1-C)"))
 (via (at 143.775 92.2) (size 0.6) (drill 0.3) (layers "F.Cu" "B.Cu") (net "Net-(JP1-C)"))
 (segment (start 143.0525 91.483) (end 143.058 91.483) (width 0.2) (layer "B.Cu") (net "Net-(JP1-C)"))
 (segment (start 143.0561 91.478) (end 143.0561 91.4811) (width 0.2) (layer "B.Cu") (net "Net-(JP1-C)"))
 (segment (start 143.058 91.483) (end 143.775 92.2) (width 0.2) (layer "B.Cu") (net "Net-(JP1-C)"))
 (segment (start 138.63 87.9) (end 137.853316 88.676684) (width 0.2) (layer "F.Cu") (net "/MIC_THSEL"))
 (segment (start 138.649496 87.9) (end 138.63 87.9) (width 0.2) (layer "F.Cu") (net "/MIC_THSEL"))
 (segment (start 137.853316 88.676684) (end 137.847504 88.676684) (width 0.2) (layer "F.Cu") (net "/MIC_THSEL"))
 (via (at 137.847504 88.676684) (size 0.6) (drill 0.3) (layers "F.Cu" "B.Cu") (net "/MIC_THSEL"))
 (segment (start 141.19 93.5) (end 139.85 93.5) (width 0.2) (layer "B.Cu") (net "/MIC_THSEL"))
 (segment (start 137.847504 91.497504) (end 137.847504 88.676684) (width 0.2) (layer "B.Cu") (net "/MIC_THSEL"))
 (segment (start 139.85 93.5) (end 137.847504 91.497504) (width 0.2) (layer "B.Cu") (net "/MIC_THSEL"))
 (segment (start 139.149622 88.450378) (end 138.825 88.775) (width 0.2) (layer "F.Cu") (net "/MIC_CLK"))
 (segment (start 138.825 88.775) (end 138.825 89.4) (width 0.2) (layer "F.Cu") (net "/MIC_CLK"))
 (segment (start 139.149622 87.900001) (end 139.149622 88.450378) (width 0.2) (layer "F.Cu") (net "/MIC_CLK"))
 (via (at 138.825 89.4) (size 0.6) (drill 0.3) (layers "F.Cu" "B.Cu") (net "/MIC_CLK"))
 (segment (start 141.3775 91.483) (end 139.558 91.483) (width 0.2) (layer "B.Cu") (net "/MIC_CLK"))
 (segment (start 139.558 91.483) (end 138.825 90.75) (width 0.2) (layer "B.Cu") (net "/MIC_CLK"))
 (segment (start 138.825 90.75) (end 138.825 89.4) (width 0.2) (layer "B.Cu") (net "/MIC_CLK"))
 (segment (start 141.3781 91.475) (end 141.3811 91.478) (width 0.2) (layer "B.Cu") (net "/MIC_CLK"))
 (segment (start 139.649748 89.05264) (end 139.649748 87.9) (width 0.2) (layer "F.Cu") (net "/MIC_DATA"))
 (segment (start 139.922108 89.325) (end 139.649748 89.05264) (width 0.2) (layer "F.Cu") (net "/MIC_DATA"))
 (segment (start 139.925 89.325) (end 139.922108 89.325) (width 0.2) (layer "F.Cu") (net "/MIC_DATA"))
 (via (at 139.925 89.325) (size 0.6) (drill 0.3) (layers "F.Cu" "B.Cu") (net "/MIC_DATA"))
 (segment (start 139.925 89.325) (end 140.425 89.825) (width 0.2) (layer "B.Cu") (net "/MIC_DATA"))
 (segment (start 140.425 89.825) (end 142.2231 89.825) (width 0.2) (layer "B.Cu") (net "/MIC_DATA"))
 (segment (start 143.0525 90.6544) (end 143.0525 90.663) (width 0.2) (layer "B.Cu") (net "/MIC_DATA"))
 (segment (start 142.2231 89.825) (end 143.0525 90.6544) (width 0.2) (layer "B.Cu") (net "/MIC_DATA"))
 (segment (start 140.149874 88.453474) (end 140.6964 89) (width 0.2) (layer "F.Cu") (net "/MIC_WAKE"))
 (segment (start 140.149874 87.900001) (end 140.149874 88.453474) (width 0.2) (layer "F.Cu") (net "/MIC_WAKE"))
 (via (at 140.6964 89) (size 0.6) (drill 0.3) (layers "F.Cu" "B.Cu") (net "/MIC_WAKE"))
 (segment (start 143.132107 89) (end 144.4 90.267893) (width 0.2) (layer "B.Cu") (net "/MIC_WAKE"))
 (segment (start 140.6964 89) (end 143.132107 89) (width 0.2) (layer "B.Cu") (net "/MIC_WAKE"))
 (segment (start 144.4 90.267893) (end 144.4 92.3386) (width 0.2) (layer "B.Cu") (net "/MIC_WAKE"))
 (segment (start 143.24 93.4986) (end 143.24 93.5) (width 0.2) (layer "B.Cu") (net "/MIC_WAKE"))
 (segment (start 144.4 92.3386) (end 143.24 93.4986) (width 0.2) (layer "B.Cu") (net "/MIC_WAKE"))
 (segment (start 140.149874 85.079126) (end 140.149874 85.512399) (width 0.2) (layer "F.Cu") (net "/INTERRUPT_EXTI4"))
 (segment (start 140.404 84.825) (end 140.149874 85.079126) (width 0.2) (layer "F.Cu") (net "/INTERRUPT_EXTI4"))
 (segment (start 142.203948 86.053948) (end 140.975 84.825) (width 0.2) (layer "F.Cu") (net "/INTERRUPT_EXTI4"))
 (segment (start 140.975 84.825) (end 140.404 84.825) (width 0.2) (layer "F.Cu") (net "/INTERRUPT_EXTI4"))
 (segment (start 142.203948 86.891468) (end 142.203948 86.053948) (width 0.2) (layer "F.Cu") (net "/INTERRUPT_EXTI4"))
 (via (at 142.203948 86.891468) (size 0.6) (drill 0.3) (layers "F.Cu" "B.Cu") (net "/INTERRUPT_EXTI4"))
 (segment (start 142.020416 87.075) (end 140.825 87.075) (width 0.2) (layer "B.Cu") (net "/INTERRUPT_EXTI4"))
 (segment (start 140.19 87.71) (end 140.19 88.18) (width 0.2) (layer "B.Cu") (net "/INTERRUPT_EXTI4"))
 (segment (start 140.825 87.075) (end 140.19 87.71) (width 0.2) (layer "B.Cu") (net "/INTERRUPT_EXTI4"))
 (segment (start 142.203948 86.891468) (end 142.020416 87.075) (width 0.2) (layer "B.Cu") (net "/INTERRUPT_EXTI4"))
 (segment (start 140.225 84.35) (end 139.649748 84.925252) (width 0.2) (layer "F.Cu") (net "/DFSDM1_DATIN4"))
 (segment (start 142.65 84.35) (end 140.225 84.35) (width 0.2) (layer "F.Cu") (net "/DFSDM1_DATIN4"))
 (segment (start 143.575 85.275) (end 142.65 84.35) (width 0.2) (layer "F.Cu") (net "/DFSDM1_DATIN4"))
 (segment (start 143.575 85.45) (end 143.575 85.275) (width 0.2) (layer "F.Cu") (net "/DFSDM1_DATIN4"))
 (segment (start 139.649748 84.925252) (end 139.649748 85.5124) (width 0.2) (layer "F.Cu") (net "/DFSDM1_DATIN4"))
 (via (at 143.575 85.45) (size 0.6) (drill 0.3) (layers "F.Cu" "B.Cu") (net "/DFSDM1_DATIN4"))
 (segment (start 139.175 86.025) (end 143.305 86.025) (width 0.2) (layer "B.Cu") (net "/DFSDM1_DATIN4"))
 (segment (start 138.99 85.47) (end 138.99 85.84) (width 0.2) (layer "B.Cu") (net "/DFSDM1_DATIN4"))
 (segment (start 143.305 86.025) (end 143.575 85.755) (width 0.2) (layer "B.Cu") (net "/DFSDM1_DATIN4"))
 (segment (start 138.99 85.84) (end 139.175 86.025) (width 0.2) (layer "B.Cu") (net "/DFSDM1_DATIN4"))
 (segment (start 143.575 85.755) (end 143.575 85.45) (width 0.2) (layer "B.Cu") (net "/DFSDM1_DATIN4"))
 (segment (start 139.149622 85.079126) (end 139.149622 85.5124) (width 0.2) (layer "F.Cu") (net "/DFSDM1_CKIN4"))
 (segment (start 138.920496 84.85) (end 139.149622 85.079126) (width 0.2) (layer "F.Cu") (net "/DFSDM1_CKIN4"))
 (segment (start 138.028554 84.85) (end 138.920496 84.85) (width 0.2) (layer "F.Cu") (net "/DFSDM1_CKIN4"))
 (via (at 138.028554 84.85) (size 0.6) (drill 0.3) (layers "F.Cu" "B.Cu") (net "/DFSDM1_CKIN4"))
 (segment (start 138.028554 84.85) (end 137.675 84.85) (width 0.2) (layer "B.Cu") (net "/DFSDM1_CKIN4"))
 (segment (start 137.675 84.85) (end 137.11 85.415) (width 0.2) (layer "B.Cu") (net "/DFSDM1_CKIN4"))
 (segment (start 137.8 87.25) (end 138.53 87.25) (width 0.2) (layer "B.Cu") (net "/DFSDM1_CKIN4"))
 (segment (start 138.99 87.71) (end 138.99 88.18) (width 0.2) (layer "B.Cu") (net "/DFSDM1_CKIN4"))
 (segment (start 137.11 85.415) (end 137.11 86.56) (width 0.2) (layer "B.Cu") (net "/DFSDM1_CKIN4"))
 (segment (start 137.11 86.56) (end 137.8 87.25) (width 0.2) (layer "B.Cu") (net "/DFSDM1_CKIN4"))
 (segment (start 138.53 87.25) (end 138.99 87.71) (width 0.2) (layer "B.Cu") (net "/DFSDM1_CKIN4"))
 (segment (start 137.61 85.76) (end 137.61 85.91) (width 0.2) (layer "F.Cu") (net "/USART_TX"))
 (segment (start 138.649496 85.5124) (end 137.8576 85.5124) (width 0.2) (layer "F.Cu") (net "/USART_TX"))
 (segment (start 137.8576 85.5124) (end 137.61 85.76) (width 0.2) (layer "F.Cu") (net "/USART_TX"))
 (via (at 137.61 85.91) (size 0.6) (drill 0.3) (layers "F.Cu" "B.Cu") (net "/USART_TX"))
 (segment (start 141.990945 86.391468) (end 141.807413 86.575) (width 0.2) (layer "B.Cu") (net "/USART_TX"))
 (segment (start 138.025 86.575) (end 137.61 86.16) (width 0.2) (layer "B.Cu") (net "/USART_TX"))
 (segment (start 142.703948 86.684361) (end 142.411055 86.391468) (width 0.2) (layer "B.Cu") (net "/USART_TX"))
 (segment (start 141.79 87.81) (end 142.208532 87.391468) (width 0.2) (layer "B.Cu") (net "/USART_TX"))
 (segment (start 142.208532 87.391468) (end 142.411055 87.391468) (width 0.2) (layer "B.Cu") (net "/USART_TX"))
 (segment (start 141.79 88.18) (end 141.79 87.81) (width 0.2) (layer "B.Cu") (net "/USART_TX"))
 (segment (start 142.411055 87.391468) (end 142.703948 87.098575) (width 0.2) (layer "B.Cu") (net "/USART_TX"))
 (segment (start 137.61 86.16) (end 137.61 85.91) (width 0.2) (layer "B.Cu") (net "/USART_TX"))
 (segment (start 142.703948 87.098575) (end 142.703948 86.684361) (width 0.2) (layer "B.Cu") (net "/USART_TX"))
 (segment (start 142.411055 86.391468) (end 141.990945 86.391468) (width 0.2) (layer "B.Cu") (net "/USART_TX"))
 (segment (start 141.807413 86.575) (end 138.025 86.575) (width 0.2) (layer "B.Cu") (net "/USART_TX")))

